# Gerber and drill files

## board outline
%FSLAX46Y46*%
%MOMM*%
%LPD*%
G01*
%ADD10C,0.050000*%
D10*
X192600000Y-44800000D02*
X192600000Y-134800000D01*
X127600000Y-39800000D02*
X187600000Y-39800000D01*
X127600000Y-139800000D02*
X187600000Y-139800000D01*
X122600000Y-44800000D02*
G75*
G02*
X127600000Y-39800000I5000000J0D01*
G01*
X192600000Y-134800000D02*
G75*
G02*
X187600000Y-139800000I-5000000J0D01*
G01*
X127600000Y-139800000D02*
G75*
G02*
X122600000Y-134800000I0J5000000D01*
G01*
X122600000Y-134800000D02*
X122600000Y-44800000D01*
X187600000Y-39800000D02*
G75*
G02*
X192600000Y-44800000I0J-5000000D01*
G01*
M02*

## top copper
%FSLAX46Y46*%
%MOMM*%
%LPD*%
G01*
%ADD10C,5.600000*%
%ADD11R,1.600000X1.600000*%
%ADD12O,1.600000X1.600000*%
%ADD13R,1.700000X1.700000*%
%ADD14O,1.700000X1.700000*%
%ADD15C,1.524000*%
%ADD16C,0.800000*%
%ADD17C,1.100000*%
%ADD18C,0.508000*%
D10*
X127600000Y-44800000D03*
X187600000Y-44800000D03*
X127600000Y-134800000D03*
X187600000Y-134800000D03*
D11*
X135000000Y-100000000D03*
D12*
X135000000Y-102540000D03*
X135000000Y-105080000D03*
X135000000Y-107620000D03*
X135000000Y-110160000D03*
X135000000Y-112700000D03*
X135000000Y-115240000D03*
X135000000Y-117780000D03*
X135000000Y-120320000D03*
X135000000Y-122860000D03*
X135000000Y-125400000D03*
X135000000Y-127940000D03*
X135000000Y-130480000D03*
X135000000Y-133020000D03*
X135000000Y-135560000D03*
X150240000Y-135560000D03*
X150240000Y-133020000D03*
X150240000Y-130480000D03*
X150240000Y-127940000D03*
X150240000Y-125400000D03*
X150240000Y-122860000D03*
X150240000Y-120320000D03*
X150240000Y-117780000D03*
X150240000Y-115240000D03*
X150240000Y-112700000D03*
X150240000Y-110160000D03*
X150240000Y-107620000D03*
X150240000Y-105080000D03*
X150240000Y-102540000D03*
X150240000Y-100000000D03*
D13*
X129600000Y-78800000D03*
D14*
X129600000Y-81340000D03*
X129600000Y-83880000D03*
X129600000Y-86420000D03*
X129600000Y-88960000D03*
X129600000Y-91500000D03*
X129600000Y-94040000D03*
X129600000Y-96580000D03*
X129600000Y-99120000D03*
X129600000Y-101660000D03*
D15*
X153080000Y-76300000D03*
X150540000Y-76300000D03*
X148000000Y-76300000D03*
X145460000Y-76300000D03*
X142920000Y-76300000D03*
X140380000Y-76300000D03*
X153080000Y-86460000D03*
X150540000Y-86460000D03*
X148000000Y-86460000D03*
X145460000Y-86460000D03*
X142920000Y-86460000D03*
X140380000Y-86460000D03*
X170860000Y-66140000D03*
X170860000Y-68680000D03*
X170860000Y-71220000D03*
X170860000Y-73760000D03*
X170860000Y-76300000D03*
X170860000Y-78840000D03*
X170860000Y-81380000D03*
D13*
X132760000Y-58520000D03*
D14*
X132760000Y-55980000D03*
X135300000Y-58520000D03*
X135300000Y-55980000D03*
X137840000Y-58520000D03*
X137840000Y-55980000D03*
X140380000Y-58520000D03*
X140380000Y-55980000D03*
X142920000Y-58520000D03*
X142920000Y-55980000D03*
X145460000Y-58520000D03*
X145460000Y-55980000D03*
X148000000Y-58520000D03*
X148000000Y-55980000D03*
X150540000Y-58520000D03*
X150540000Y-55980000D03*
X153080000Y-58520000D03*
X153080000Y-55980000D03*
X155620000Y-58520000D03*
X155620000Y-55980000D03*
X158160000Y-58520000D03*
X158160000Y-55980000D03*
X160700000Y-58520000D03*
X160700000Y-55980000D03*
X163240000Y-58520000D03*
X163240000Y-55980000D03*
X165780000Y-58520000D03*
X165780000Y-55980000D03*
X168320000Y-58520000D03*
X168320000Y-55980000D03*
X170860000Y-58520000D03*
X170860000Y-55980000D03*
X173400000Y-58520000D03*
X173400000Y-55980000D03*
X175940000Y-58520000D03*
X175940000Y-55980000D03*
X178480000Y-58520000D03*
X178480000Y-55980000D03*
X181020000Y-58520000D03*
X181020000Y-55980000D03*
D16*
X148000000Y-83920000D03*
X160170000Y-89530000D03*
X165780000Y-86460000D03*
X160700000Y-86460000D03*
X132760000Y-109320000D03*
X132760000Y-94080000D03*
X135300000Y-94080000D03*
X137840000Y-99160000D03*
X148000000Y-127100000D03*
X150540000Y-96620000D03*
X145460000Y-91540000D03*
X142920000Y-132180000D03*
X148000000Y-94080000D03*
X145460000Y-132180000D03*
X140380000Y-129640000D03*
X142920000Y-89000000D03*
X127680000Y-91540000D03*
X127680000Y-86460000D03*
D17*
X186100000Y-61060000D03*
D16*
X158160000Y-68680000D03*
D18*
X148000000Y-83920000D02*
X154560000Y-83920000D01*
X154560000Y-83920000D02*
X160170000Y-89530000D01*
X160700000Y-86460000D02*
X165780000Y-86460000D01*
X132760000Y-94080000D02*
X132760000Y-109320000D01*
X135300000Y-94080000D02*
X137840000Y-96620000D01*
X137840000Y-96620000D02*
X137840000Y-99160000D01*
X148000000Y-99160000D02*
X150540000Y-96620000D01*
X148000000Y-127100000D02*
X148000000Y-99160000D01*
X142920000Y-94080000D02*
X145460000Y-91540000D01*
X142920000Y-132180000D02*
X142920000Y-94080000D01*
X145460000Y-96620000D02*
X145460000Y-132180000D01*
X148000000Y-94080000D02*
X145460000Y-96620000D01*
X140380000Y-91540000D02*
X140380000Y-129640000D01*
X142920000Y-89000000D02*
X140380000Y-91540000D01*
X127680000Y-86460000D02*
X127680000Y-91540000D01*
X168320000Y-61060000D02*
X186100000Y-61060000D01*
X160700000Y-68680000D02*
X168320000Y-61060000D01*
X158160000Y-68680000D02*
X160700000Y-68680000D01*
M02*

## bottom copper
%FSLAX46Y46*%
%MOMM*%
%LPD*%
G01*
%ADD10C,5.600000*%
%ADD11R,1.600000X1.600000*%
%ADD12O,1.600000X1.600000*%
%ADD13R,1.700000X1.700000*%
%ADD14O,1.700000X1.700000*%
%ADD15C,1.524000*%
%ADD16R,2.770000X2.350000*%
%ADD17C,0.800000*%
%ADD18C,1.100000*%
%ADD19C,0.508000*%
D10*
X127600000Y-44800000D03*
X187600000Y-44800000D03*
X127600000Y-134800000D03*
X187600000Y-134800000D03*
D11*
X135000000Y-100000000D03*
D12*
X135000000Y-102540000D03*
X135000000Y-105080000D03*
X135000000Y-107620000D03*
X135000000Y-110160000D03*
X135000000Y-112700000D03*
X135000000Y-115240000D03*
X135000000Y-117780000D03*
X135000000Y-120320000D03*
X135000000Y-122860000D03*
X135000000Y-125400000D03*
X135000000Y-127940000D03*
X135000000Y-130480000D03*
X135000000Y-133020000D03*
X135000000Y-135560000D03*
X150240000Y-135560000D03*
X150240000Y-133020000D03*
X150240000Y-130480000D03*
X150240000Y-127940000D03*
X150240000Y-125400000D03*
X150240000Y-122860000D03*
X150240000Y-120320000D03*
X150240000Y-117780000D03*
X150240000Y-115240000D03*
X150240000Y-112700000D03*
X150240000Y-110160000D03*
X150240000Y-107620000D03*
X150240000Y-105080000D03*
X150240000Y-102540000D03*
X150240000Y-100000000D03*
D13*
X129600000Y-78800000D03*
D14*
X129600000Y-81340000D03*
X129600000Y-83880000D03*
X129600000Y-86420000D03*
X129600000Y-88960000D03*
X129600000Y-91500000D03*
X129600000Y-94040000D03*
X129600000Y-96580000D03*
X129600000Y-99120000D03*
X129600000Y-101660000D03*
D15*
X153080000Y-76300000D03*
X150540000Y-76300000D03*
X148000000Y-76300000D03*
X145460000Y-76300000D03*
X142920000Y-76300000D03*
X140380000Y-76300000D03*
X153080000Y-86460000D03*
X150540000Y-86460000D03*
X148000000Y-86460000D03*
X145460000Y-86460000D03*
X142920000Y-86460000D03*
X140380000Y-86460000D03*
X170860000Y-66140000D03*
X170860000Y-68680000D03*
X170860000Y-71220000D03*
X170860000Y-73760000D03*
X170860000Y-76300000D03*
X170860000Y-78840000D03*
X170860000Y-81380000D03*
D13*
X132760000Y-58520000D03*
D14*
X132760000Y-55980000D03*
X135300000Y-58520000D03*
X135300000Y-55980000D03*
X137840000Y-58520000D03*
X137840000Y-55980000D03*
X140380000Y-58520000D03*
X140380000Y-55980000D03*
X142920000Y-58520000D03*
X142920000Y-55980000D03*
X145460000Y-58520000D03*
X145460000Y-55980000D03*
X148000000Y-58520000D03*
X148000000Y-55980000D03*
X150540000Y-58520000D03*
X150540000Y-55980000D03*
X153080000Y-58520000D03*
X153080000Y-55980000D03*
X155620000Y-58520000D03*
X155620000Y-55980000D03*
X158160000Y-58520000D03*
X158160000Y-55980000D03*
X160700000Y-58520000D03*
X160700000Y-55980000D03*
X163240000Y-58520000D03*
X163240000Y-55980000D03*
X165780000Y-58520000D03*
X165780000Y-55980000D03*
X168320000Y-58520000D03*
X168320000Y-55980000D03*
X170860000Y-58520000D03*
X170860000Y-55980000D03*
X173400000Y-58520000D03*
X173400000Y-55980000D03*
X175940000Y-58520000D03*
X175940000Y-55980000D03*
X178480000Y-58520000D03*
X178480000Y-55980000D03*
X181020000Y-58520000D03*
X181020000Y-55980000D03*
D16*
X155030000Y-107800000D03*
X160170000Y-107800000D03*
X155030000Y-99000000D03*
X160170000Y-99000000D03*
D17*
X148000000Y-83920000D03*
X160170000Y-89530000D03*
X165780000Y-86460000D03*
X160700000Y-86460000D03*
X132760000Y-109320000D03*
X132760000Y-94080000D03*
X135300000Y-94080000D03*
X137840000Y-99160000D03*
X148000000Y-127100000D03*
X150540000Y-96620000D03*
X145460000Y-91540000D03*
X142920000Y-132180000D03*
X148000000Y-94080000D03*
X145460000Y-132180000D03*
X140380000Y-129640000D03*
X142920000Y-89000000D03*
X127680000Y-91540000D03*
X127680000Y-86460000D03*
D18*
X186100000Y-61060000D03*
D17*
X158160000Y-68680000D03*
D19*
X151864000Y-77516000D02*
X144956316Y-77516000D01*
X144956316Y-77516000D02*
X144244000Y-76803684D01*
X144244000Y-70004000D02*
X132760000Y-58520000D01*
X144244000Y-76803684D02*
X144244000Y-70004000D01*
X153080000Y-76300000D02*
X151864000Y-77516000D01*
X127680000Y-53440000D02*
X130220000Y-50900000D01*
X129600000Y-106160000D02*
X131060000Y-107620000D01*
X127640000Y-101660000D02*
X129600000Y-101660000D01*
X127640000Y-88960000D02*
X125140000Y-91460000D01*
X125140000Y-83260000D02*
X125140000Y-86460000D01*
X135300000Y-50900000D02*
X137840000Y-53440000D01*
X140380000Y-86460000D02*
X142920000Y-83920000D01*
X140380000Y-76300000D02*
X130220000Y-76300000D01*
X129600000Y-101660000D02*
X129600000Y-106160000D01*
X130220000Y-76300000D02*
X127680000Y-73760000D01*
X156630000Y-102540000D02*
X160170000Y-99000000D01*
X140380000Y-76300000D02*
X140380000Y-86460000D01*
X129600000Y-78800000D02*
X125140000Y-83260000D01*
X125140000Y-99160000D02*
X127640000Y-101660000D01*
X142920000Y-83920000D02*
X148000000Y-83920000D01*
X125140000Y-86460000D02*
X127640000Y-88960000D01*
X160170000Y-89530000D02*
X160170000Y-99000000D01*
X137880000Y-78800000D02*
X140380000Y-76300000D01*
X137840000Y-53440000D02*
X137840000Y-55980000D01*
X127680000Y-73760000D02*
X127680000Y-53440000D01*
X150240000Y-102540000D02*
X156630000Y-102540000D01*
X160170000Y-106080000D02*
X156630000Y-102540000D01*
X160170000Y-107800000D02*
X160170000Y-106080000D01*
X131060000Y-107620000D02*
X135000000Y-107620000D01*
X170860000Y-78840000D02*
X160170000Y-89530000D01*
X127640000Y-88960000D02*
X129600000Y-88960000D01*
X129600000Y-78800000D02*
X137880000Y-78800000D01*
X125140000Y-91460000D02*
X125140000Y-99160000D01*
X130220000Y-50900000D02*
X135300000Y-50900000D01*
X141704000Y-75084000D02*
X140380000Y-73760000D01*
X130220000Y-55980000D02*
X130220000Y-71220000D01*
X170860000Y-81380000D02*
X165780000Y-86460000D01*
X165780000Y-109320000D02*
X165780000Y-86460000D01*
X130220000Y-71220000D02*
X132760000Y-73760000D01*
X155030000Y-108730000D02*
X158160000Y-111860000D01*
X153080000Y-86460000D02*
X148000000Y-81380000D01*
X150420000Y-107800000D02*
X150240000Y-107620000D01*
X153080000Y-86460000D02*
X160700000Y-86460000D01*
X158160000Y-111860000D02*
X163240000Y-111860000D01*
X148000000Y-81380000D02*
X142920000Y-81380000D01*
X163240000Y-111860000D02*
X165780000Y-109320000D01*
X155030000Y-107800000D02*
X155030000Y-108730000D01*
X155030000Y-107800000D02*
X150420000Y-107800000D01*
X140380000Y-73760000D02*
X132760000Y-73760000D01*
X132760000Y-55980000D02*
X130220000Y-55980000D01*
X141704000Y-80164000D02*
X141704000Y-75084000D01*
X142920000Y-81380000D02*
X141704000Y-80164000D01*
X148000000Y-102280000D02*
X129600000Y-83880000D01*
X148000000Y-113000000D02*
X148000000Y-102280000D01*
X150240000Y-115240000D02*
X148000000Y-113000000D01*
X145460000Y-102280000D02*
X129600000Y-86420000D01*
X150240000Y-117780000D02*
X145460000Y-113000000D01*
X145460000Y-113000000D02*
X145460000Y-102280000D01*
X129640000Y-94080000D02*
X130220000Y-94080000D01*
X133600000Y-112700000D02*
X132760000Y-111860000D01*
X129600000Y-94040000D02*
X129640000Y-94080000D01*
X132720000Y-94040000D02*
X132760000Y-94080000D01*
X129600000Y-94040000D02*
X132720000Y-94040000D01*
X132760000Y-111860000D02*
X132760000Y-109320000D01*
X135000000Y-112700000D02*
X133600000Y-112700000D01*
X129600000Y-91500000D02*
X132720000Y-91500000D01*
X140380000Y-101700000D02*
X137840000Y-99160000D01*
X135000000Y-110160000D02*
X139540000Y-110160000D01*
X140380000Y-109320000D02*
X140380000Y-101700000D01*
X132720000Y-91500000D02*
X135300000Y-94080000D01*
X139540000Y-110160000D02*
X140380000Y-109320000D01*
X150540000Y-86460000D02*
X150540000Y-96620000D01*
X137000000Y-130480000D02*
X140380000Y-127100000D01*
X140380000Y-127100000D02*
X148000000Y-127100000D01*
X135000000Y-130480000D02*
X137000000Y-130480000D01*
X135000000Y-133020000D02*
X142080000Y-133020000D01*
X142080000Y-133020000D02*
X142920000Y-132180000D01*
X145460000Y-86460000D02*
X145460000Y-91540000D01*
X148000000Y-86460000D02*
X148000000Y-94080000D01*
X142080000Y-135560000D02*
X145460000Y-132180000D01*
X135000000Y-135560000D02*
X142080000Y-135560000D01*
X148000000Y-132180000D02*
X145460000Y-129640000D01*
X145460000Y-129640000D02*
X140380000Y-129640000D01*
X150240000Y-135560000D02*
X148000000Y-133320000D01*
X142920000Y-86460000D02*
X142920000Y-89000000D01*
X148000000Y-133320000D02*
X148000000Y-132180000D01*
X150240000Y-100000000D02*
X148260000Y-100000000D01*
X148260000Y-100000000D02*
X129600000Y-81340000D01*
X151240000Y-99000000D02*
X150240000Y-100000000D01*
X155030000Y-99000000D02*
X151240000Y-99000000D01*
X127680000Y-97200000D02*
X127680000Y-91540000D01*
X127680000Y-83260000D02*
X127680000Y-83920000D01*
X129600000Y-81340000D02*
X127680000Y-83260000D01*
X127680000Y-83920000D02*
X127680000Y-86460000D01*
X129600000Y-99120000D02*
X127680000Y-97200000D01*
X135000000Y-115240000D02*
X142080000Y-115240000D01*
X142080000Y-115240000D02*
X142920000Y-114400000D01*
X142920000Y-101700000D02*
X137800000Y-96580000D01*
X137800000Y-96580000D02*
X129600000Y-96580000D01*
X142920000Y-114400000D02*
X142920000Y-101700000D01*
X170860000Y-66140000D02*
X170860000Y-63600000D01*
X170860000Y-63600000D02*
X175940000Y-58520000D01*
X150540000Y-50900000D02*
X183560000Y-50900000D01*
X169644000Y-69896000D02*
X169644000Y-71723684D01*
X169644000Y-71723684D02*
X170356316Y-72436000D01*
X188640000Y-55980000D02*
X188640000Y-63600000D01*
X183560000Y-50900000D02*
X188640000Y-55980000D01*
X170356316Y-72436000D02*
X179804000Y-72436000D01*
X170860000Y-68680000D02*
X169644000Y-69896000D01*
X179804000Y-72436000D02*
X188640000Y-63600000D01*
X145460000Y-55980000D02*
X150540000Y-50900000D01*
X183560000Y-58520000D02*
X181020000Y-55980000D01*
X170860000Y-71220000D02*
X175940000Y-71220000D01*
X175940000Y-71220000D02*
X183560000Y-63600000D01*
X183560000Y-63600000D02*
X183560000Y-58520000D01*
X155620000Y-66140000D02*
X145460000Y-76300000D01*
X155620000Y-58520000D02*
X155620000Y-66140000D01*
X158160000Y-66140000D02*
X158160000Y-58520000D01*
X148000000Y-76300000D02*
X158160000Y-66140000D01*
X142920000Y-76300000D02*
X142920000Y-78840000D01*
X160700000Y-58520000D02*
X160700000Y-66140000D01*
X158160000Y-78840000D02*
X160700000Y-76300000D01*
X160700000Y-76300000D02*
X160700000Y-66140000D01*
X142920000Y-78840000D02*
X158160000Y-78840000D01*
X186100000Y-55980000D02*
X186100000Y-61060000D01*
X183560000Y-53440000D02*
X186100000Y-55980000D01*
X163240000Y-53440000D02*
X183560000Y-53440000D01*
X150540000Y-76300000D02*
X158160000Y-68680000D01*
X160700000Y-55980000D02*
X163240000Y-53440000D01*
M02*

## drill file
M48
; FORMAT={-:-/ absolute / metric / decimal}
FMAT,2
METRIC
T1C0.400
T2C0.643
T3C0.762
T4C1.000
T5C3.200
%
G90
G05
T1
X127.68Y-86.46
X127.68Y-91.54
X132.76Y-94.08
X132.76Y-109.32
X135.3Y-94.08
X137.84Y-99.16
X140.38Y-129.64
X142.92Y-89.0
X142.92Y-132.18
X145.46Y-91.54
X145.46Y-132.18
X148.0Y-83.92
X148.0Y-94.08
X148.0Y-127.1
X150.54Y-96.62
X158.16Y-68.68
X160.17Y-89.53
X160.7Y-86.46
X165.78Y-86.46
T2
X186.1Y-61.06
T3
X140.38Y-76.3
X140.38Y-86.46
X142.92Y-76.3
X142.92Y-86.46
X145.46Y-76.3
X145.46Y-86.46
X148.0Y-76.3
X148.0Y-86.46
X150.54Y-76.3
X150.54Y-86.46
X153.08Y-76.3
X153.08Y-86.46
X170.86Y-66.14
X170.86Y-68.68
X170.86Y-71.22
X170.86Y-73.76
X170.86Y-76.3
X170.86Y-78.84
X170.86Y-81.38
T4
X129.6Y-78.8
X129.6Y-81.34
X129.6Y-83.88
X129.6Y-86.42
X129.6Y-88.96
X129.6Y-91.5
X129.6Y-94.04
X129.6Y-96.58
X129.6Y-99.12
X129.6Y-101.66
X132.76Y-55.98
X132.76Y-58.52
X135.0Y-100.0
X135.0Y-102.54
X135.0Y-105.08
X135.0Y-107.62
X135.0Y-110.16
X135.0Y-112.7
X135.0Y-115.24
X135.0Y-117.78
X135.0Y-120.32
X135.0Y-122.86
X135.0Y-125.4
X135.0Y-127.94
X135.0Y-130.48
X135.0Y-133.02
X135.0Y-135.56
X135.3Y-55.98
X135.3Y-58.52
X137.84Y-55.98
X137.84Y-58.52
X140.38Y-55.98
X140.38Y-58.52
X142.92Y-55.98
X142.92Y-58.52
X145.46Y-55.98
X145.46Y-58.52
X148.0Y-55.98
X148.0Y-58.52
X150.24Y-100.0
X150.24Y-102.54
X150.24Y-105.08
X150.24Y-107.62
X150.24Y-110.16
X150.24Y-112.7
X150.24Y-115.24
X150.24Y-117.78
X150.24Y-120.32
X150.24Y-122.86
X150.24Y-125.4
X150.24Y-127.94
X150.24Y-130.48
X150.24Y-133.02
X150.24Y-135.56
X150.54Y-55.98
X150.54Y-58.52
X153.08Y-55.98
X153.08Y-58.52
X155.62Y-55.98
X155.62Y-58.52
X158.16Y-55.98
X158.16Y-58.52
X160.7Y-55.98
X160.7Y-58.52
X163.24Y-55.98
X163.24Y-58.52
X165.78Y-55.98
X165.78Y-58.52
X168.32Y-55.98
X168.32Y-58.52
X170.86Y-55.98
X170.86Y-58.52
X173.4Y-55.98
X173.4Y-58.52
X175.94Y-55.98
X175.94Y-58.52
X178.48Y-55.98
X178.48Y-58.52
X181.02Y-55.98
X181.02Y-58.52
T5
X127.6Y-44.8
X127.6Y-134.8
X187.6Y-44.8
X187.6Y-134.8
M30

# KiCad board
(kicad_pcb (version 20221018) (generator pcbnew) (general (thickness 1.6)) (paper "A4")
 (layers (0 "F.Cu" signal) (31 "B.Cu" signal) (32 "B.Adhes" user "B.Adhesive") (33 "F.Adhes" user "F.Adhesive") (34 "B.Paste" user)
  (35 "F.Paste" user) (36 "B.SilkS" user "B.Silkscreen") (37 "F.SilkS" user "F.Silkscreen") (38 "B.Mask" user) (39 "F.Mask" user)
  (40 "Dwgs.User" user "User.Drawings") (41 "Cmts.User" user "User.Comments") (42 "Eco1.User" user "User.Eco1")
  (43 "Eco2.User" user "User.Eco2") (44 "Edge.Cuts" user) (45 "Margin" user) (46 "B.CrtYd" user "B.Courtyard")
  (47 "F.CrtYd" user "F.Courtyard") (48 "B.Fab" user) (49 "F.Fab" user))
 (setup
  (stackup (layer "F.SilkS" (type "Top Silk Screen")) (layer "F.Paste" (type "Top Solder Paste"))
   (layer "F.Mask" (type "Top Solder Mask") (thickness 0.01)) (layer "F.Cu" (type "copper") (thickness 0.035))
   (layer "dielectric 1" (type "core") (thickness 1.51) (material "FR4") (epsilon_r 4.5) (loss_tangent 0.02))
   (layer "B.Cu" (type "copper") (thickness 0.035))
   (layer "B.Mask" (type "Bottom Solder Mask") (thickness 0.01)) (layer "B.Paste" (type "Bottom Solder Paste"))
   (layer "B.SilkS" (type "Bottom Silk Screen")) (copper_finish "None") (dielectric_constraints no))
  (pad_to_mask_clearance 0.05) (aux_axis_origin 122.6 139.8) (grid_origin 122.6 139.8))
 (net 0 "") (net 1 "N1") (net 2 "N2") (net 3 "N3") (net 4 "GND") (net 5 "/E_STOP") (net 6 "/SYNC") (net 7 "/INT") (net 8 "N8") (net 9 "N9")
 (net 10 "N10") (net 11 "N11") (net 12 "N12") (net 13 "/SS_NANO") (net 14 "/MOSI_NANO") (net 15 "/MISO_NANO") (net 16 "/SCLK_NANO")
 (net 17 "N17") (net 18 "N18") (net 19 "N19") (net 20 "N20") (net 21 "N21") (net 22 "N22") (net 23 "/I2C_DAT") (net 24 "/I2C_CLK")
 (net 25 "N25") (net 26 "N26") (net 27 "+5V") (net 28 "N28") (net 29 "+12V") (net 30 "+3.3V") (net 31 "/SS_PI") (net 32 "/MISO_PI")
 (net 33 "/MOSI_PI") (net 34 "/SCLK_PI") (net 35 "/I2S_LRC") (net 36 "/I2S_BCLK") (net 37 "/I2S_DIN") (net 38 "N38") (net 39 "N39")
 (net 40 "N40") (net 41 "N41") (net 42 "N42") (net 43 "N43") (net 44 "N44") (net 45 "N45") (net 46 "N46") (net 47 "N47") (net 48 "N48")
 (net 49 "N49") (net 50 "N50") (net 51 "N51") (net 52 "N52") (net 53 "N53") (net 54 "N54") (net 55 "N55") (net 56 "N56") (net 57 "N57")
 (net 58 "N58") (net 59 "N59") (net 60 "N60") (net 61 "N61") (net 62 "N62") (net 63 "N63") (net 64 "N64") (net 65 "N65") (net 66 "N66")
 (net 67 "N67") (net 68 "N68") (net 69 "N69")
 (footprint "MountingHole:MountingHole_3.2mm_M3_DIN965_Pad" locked (layer "F.Cu") (at 127.6 44.8)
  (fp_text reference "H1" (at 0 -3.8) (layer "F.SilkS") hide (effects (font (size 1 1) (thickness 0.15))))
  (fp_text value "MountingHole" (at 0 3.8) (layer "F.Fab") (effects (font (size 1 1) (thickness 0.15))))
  (pad "1" thru_hole circle locked (at 0 0) (size 5.6 5.6) (drill 3.2) (layers "*.Cu" "*.Mask")))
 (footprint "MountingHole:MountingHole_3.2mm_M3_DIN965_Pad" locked (layer "F.Cu") (at 187.6 44.8)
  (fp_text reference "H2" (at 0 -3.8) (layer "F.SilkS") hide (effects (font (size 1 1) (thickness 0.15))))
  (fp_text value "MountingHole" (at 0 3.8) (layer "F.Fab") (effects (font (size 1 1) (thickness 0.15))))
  (pad "1" thru_hole circle locked (at 0 0) (size 5.6 5.6) (drill 3.2) (layers "*.Cu" "*.Mask")))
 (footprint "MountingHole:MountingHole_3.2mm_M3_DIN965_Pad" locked (layer "F.Cu") (at 127.6 134.8)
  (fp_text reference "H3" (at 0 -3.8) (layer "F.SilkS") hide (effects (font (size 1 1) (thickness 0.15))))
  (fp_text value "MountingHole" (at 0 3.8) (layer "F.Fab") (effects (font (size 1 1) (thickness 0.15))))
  (pad "1" thru_hole circle locked (at 0 0) (size 5.6 5.6) (drill 3.2) (layers "*.Cu" "*.Mask")))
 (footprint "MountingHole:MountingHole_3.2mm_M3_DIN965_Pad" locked (layer "F.Cu") (at 187.6 134.8)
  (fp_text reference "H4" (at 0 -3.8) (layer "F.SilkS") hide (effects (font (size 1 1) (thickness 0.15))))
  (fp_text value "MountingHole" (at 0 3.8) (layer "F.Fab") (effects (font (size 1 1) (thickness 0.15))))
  (pad "1" thru_hole circle locked (at 0 0) (size 5.6 5.6) (drill 3.2) (layers "*.Cu" "*.Mask")))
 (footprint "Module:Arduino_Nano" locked (layer "F.Cu") (at 135 100)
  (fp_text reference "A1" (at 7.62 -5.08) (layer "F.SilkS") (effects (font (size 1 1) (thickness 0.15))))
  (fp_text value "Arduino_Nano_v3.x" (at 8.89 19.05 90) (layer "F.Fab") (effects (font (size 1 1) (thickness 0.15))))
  (pad "1" thru_hole rect locked (at 0 0) (size 1.6 1.6) (drill 1) (layers "*.Cu" "*.Mask") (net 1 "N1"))
  (pad "2" thru_hole oval locked (at 0 2.54) (size 1.6 1.6) (drill 1) (layers "*.Cu" "*.Mask") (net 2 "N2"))
  (pad "3" thru_hole oval locked (at 0 5.08) (size 1.6 1.6) (drill 1) (layers "*.Cu" "*.Mask") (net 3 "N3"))
  (pad "4" thru_hole oval locked (at 0 7.62) (size 1.6 1.6) (drill 1) (layers "*.Cu" "*.Mask") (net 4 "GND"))
  (pad "5" thru_hole oval locked (at 0 10.16) (size 1.6 1.6) (drill 1) (layers "*.Cu" "*.Mask") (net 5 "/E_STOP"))
  (pad "6" thru_hole oval locked (at 0 12.7) (size 1.6 1.6) (drill 1) (layers "*.Cu" "*.Mask") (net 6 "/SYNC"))
  (pad "7" thru_hole oval locked (at 0 15.24) (size 1.6 1.6) (drill 1) (layers "*.Cu" "*.Mask") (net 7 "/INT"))
  (pad "8" thru_hole oval locked (at 0 17.78) (size 1.6 1.6) (drill 1) (layers "*.Cu" "*.Mask") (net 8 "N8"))
  (pad "9" thru_hole oval locked (at 0 20.32) (size 1.6 1.6) (drill 1) (layers "*.Cu" "*.Mask") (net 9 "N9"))
  (pad "10" thru_hole oval locked (at 0 22.86) (size 1.6 1.6) (drill 1) (layers "*.Cu" "*.Mask") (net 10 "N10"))
  (pad "11" thru_hole oval locked (at 0 25.4) (size 1.6 1.6) (drill 1) (layers "*.Cu" "*.Mask") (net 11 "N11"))
  (pad "12" thru_hole oval locked (at 0 27.94) (size 1.6 1.6) (drill 1) (layers "*.Cu" "*.Mask") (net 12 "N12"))
  (pad "13" thru_hole oval locked (at 0 30.48) (size 1.6 1.6) (drill 1) (layers "*.Cu" "*.Mask") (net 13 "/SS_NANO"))
  (pad "14" thru_hole oval locked (at 0 33.02) (size 1.6 1.6) (drill 1) (layers "*.Cu" "*.Mask") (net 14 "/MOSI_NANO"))
  (pad "15" thru_hole oval locked (at 0 35.56) (size 1.6 1.6) (drill 1) (layers "*.Cu" "*.Mask") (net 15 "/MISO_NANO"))
  (pad "16" thru_hole oval locked (at 15.24 35.56) (size 1.6 1.6) (drill 1) (layers "*.Cu" "*.Mask") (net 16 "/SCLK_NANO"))
  (pad "17" thru_hole oval locked (at 15.24 33.02) (size 1.6 1.6) (drill 1) (layers "*.Cu" "*.Mask") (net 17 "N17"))
  (pad "18" thru_hole oval locked (at 15.24 30.48) (size 1.6 1.6) (drill 1) (layers "*.Cu" "*.Mask") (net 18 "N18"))
  (pad "19" thru_hole oval locked (at 15.24 27.94) (size 1.6 1.6) (drill 1) (layers "*.Cu" "*.Mask") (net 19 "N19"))
  (pad "20" thru_hole oval locked (at 15.24 25.4) (size 1.6 1.6) (drill 1) (layers "*.Cu" "*.Mask") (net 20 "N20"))
  (pad "21" thru_hole oval locked (at 15.24 22.86) (size 1.6 1.6) (drill 1) (layers "*.Cu" "*.Mask") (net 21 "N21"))
  (pad "22" thru_hole oval locked (at 15.24 20.32) (size 1.6 1.6) (drill 1) (layers "*.Cu" "*.Mask") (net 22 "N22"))
  (pad "23" thru_hole oval locked (at 15.24 17.78) (size 1.6 1.6) (drill 1) (layers "*.Cu" "*.Mask") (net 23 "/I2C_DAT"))
  (pad "24" thru_hole oval locked (at 15.24 15.24) (size 1.6 1.6) (drill 1) (layers "*.Cu" "*.Mask") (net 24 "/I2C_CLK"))
  (pad "25" thru_hole oval locked (at 15.24 12.7) (size 1.6 1.6) (drill 1) (layers "*.Cu" "*.Mask") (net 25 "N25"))
  (pad "26" thru_hole oval locked (at 15.24 10.16) (size 1.6 1.6) (drill 1) (layers "*.Cu" "*.Mask") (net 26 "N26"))
  (pad "27" thru_hole oval locked (at 15.24 7.62) (size 1.6 1.6) (drill 1) (layers "*.Cu" "*.Mask") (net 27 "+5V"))
  (pad "28" thru_hole oval locked (at 15.24 5.08) (size 1.6 1.6) (drill 1) (layers "*.Cu" "*.Mask") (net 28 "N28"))
  (pad "29" thru_hole oval locked (at 15.24 2.54) (size 1.6 1.6) (drill 1) (layers "*.Cu" "*.Mask") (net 4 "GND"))
  (pad "30" thru_hole oval locked (at 15.24 0) (size 1.6 1.6) (drill 1) (layers "*.Cu" "*.Mask") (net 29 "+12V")))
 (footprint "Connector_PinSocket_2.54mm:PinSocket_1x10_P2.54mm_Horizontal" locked (layer "F.Cu") (at 129.6 78.8)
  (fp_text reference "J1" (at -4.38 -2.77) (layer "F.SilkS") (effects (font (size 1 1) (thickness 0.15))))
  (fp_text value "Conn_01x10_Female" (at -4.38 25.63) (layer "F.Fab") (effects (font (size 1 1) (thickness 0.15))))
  (pad "1" thru_hole rect locked (at 0 0) (size 1.7 1.7) (drill 1) (layers "*.Cu" "*.Mask") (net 4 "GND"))
  (pad "2" thru_hole oval locked (at 0 2.54) (size 1.7 1.7) (drill 1) (layers "*.Cu" "*.Mask") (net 29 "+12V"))
  (pad "3" thru_hole oval locked (at 0 5.08) (size 1.7 1.7) (drill 1) (layers "*.Cu" "*.Mask") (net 24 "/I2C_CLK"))
  (pad "4" thru_hole oval locked (at 0 7.62) (size 1.7 1.7) (drill 1) (layers "*.Cu" "*.Mask") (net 23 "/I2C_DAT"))
  (pad "5" thru_hole oval locked (at 0 10.16) (size 1.7 1.7) (drill 1) (layers "*.Cu" "*.Mask") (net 4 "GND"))
  (pad "6" thru_hole oval locked (at 0 12.7) (size 1.7 1.7) (drill 1) (layers "*.Cu" "*.Mask") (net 5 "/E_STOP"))
  (pad "7" thru_hole oval locked (at 0 15.24) (size 1.7 1.7) (drill 1) (layers "*.Cu" "*.Mask") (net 6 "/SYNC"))
  (pad "8" thru_hole oval locked (at 0 17.78) (size 1.7 1.7) (drill 1) (layers "*.Cu" "*.Mask") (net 7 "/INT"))
  (pad "9" thru_hole oval locked (at 0 20.32) (size 1.7 1.7) (drill 1) (layers "*.Cu" "*.Mask") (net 29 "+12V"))
  (pad "10" thru_hole oval locked (at 0 22.86) (size 1.7 1.7) (drill 1) (layers "*.Cu" "*.Mask") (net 4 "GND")))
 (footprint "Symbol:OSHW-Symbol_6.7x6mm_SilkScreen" (layer "F.Cu") (at 166.6 135.8)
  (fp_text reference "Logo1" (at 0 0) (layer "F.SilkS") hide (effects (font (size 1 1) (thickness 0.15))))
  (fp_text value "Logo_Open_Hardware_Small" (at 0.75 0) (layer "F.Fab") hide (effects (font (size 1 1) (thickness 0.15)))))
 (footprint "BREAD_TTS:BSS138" (layer "F.Cu") (at 145.46 73.76 180)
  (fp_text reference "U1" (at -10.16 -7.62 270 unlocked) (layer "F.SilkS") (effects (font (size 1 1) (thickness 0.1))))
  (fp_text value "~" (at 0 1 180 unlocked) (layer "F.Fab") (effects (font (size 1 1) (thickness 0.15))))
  (pad "1" thru_hole circle (at -7.62 -2.54 180) (size 1.524 1.524) (drill 0.762) (layers "*.Cu" "*.Mask") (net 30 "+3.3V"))
  (pad "2" thru_hole circle (at -5.08 -2.54 180) (size 1.524 1.524) (drill 0.762) (layers "*.Cu" "*.Mask") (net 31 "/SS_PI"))
  (pad "3" thru_hole circle (at -2.54 -2.54 180) (size 1.524 1.524) (drill 0.762) (layers "*.Cu" "*.Mask") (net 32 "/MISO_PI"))
  (pad "4" thru_hole circle (at 0 -2.54 180) (size 1.524 1.524) (drill 0.762) (layers "*.Cu" "*.Mask") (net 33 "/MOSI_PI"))
  (pad "5" thru_hole circle (at 2.54 -2.54 180) (size 1.524 1.524) (drill 0.762) (layers "*.Cu" "*.Mask") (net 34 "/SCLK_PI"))
  (pad "6" thru_hole circle (at 5.08 -2.54 180) (size 1.524 1.524) (drill 0.762) (layers "*.Cu" "*.Mask") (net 4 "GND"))
  (pad "7" thru_hole circle (at -7.62 -12.7 180) (size 1.524 1.524) (drill 0.762) (layers "*.Cu" "*.Mask") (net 27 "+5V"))
  (pad "8" thru_hole circle (at -5.08 -12.7 180) (size 1.524 1.524) (drill 0.762) (layers "*.Cu" "*.Mask") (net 13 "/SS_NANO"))
  (pad "9" thru_hole circle (at -2.54 -12.7 180) (size 1.524 1.524) (drill 0.762) (layers "*.Cu" "*.Mask") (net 15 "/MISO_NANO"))
  (pad "10" thru_hole circle (at 0 -12.7 180) (size 1.524 1.524) (drill 0.762) (layers "*.Cu" "*.Mask") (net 14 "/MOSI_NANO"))
  (pad "11" thru_hole circle (at 2.54 -12.7 180) (size 1.524 1.524) (drill 0.762) (layers "*.Cu" "*.Mask") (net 16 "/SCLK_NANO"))
  (pad "12" thru_hole circle (at 5.08 -12.7 180) (size 1.524 1.524) (drill 0.762) (layers "*.Cu" "*.Mask") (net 4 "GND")))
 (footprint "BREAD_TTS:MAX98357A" (layer "F.Cu") (at 168.32 73.76 -90)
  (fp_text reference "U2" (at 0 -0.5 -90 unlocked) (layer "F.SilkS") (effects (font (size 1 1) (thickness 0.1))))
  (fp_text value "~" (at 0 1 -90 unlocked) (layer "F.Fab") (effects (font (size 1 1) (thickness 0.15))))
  (pad "1" thru_hole circle (at -7.62 -2.54 270) (size 1.524 1.524) (drill 0.762) (layers "*.Cu" "*.Mask") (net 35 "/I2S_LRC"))
  (pad "2" thru_hole circle (at -5.08 -2.54 270) (size 1.524 1.524) (drill 0.762) (layers "*.Cu" "*.Mask") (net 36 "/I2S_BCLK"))
  (pad "3" thru_hole circle (at -2.54 -2.54 270) (size 1.524 1.524) (drill 0.762) (layers "*.Cu" "*.Mask") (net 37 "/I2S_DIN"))
  (pad "4" thru_hole circle (at 0 -2.54 270) (size 1.524 1.524) (drill 0.762) (layers "*.Cu" "*.Mask") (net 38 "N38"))
  (pad "5" thru_hole circle (at 2.54 -2.54 270) (size 1.524 1.524) (drill 0.762) (layers "*.Cu" "*.Mask") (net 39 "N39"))
  (pad "6" thru_hole circle (at 5.08 -2.54 270) (size 1.524 1.524) (drill 0.762) (layers "*.Cu" "*.Mask") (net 4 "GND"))
  (pad "7" thru_hole circle (at 7.62 -2.54 270) (size 1.524 1.524) (drill 0.762) (layers "*.Cu" "*.Mask") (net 27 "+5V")))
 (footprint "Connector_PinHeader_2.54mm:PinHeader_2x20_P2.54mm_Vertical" (layer "F.Cu") (at 132.76 58.52 90)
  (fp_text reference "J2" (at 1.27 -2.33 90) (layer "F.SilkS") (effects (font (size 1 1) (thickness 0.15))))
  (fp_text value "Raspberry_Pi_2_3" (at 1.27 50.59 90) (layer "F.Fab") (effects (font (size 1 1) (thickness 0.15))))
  (pad "1" thru_hole rect (at 0 0 90) (size 1.7 1.7) (drill 1) (layers "*.Cu" "*.Mask") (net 30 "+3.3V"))
  (pad "2" thru_hole oval (at 2.54 0 90) (size 1.7 1.7) (drill 1) (layers "*.Cu" "*.Mask") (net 27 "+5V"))
  (pad "3" thru_hole oval (at 0 2.54 90) (size 1.7 1.7) (drill 1) (layers "*.Cu" "*.Mask") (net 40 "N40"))
  (pad "4" thru_hole oval (at 2.54 2.54 90) (size 1.7 1.7) (drill 1) (layers "*.Cu" "*.Mask") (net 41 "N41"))
  (pad "5" thru_hole oval (at 0 5.08 90) (size 1.7 1.7) (drill 1) (layers "*.Cu" "*.Mask") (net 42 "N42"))
  (pad "6" thru_hole oval (at 2.54 5.08 90) (size 1.7 1.7) (drill 1) (layers "*.Cu" "*.Mask") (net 4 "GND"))
  (pad "7" thru_hole oval (at 0 7.62 90) (size 1.7 1.7) (drill 1) (layers "*.Cu" "*.Mask") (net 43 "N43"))
  (pad "8" thru_hole oval (at 2.54 7.62 90) (size 1.7 1.7) (drill 1) (layers "*.Cu" "*.Mask") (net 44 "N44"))
  (pad "9" thru_hole oval (at 0 10.16 90) (size 1.7 1.7) (drill 1) (layers "*.Cu" "*.Mask") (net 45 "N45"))
  (pad "10" thru_hole oval (at 2.54 10.16 90) (size 1.7 1.7) (drill 1) (layers "*.Cu" "*.Mask") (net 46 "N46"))
  (pad "11" thru_hole oval (at 0 12.7 90) (size 1.7 1.7) (drill 1) (layers "*.Cu" "*.Mask") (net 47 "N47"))
  (pad "12" thru_hole oval (at 2.54 12.7 90) (size 1.7 1.7) (drill 1) (layers "*.Cu" "*.Mask") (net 36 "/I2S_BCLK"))
  (pad "13" thru_hole oval (at 0 15.24 90) (size 1.7 1.7) (drill 1) (layers "*.Cu" "*.Mask") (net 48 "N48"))
  (pad "14" thru_hole oval (at 2.54 15.24 90) (size 1.7 1.7) (drill 1) (layers "*.Cu" "*.Mask") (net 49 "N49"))
  (pad "15" thru_hole oval (at 0 17.78 90) (size 1.7 1.7) (drill 1) (layers "*.Cu" "*.Mask") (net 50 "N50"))
  (pad "16" thru_hole oval (at 2.54 17.78 90) (size 1.7 1.7) (drill 1) (layers "*.Cu" "*.Mask") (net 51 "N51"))
  (pad "17" thru_hole oval (at 0 20.32 90) (size 1.7 1.7) (drill 1) (layers "*.Cu" "*.Mask") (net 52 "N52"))
  (pad "18" thru_hole oval (at 2.54 20.32 90) (size 1.7 1.7) (drill 1) (layers "*.Cu" "*.Mask") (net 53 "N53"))
  (pad "19" thru_hole oval (at 0 22.86 90) (size 1.7 1.7) (drill 1) (layers "*.Cu" "*.Mask") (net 33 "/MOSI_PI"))
  (pad "20" thru_hole oval (at 2.54 22.86 90) (size 1.7 1.7) (drill 1) (layers "*.Cu" "*.Mask") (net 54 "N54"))
  (pad "21" thru_hole oval (at 0 25.4 90) (size 1.7 1.7) (drill 1) (layers "*.Cu" "*.Mask") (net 32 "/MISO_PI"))
  (pad "22" thru_hole oval (at 2.54 25.4 90) (size 1.7 1.7) (drill 1) (layers "*.Cu" "*.Mask") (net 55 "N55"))
  (pad "23" thru_hole oval (at 0 27.94 90) (size 1.7 1.7) (drill 1) (layers "*.Cu" "*.Mask") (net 34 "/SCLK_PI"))
  (pad "24" thru_hole oval (at 2.54 27.94 90) (size 1.7 1.7) (drill 1) (layers "*.Cu" "*.Mask") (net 31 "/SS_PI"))
  (pad "25" thru_hole oval (at 0 30.48 90) (size 1.7 1.7) (drill 1) (layers "*.Cu" "*.Mask") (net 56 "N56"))
  (pad "26" thru_hole oval (at 2.54 30.48 90) (size 1.7 1.7) (drill 1) (layers "*.Cu" "*.Mask") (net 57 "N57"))
  (pad "27" thru_hole oval (at 0 33.02 90) (size 1.7 1.7) (drill 1) (layers "*.Cu" "*.Mask") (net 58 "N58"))
  (pad "28" thru_hole oval (at 2.54 33.02 90) (size 1.7 1.7) (drill 1) (layers "*.Cu" "*.Mask") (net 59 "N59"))
  (pad "29" thru_hole oval (at 0 35.56 90) (size 1.7 1.7) (drill 1) (layers "*.Cu" "*.Mask") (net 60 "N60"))
  (pad "30" thru_hole oval (at 2.54 35.56 90) (size 1.7 1.7) (drill 1) (layers "*.Cu" "*.Mask") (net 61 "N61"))
  (pad "31" thru_hole oval (at 0 38.1 90) (size 1.7 1.7) (drill 1) (layers "*.Cu" "*.Mask") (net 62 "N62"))
  (pad "32" thru_hole oval (at 2.54 38.1 90) (size 1.7 1.7) (drill 1) (layers "*.Cu" "*.Mask") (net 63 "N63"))
  (pad "33" thru_hole oval (at 0 40.64 90) (size 1.7 1.7) (drill 1) (layers "*.Cu" "*.Mask") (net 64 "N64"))
  (pad "34" thru_hole oval (at 2.54 40.64 90) (size 1.7 1.7) (drill 1) (layers "*.Cu" "*.Mask") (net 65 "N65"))
  (pad "35" thru_hole oval (at 0 43.18 90) (size 1.7 1.7) (drill 1) (layers "*.Cu" "*.Mask") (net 35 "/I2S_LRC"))
  (pad "36" thru_hole oval (at 2.54 43.18 90) (size 1.7 1.7) (drill 1) (layers "*.Cu" "*.Mask") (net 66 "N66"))
  (pad "37" thru_hole oval (at 0 45.72 90) (size 1.7 1.7) (drill 1) (layers "*.Cu" "*.Mask") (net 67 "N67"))
  (pad "38" thru_hole oval (at 2.54 45.72 90) (size 1.7 1.7) (drill 1) (layers "*.Cu" "*.Mask") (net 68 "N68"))
  (pad "39" thru_hole oval (at 0 48.26 90) (size 1.7 1.7) (drill 1) (layers "*.Cu" "*.Mask") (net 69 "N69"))
  (pad "40" thru_hole oval (at 2.54 48.26 90) (size 1.7 1.7) (drill 1) (layers "*.Cu" "*.Mask") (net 37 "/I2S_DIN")))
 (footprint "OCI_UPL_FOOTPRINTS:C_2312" (layer "B.Cu") (at 157.6 107.8)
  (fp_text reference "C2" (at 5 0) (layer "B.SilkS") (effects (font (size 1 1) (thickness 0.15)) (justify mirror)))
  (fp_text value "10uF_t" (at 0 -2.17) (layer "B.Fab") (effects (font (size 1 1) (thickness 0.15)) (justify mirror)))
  (pad "1" smd rect (at -2.57 0) (size 2.77 2.35) (layers "B.Cu" "B.Paste" "B.Mask") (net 27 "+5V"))
  (pad "2" smd rect (at 2.57 0) (size 2.77 2.35) (layers "B.Cu" "B.Paste" "B.Mask") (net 4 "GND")))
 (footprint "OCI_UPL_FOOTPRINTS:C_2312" (layer "B.Cu") (at 157.6 99)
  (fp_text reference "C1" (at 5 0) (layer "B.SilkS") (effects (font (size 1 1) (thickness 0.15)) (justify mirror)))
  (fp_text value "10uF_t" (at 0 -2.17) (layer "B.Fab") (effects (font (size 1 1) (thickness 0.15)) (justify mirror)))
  (pad "1" smd rect (at -2.57 0) (size 2.77 2.35) (layers "B.Cu" "B.Paste" "B.Mask") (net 29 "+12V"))
  (pad "2" smd rect (at 2.57 0) (size 2.77 2.35) (layers "B.Cu" "B.Paste" "B.Mask") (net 4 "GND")))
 (gr_line (start 192.6 44.8) (end 192.6 134.8) (stroke (width 0.05) (type solid)) (layer "Edge.Cuts"))
 (gr_line (start 127.6 39.8) (end 187.6 39.8) (stroke (width 0.05) (type solid)) (layer "Edge.Cuts"))
 (gr_line (start 127.6 139.8) (end 187.6 139.8) (stroke (width 0.05) (type solid)) (layer "Edge.Cuts"))
 (gr_arc (start 122.6 44.8) (mid 124.064466 41.264466) (end 127.6 39.8) (stroke (width 0.05) (type solid)) (layer "Edge.Cuts"))
 (gr_arc (start 192.6 134.8) (mid 191.135534 138.335534) (end 187.6 139.8) (stroke (width 0.05) (type solid)) (layer "Edge.Cuts"))
 (gr_arc (start 127.6 139.8) (mid 124.064466 138.335534) (end 122.6 134.8) (stroke (width 0.05) (type solid)) (layer "Edge.Cuts"))
 (gr_line (start 122.6 134.8) (end 122.6 44.8) (stroke (width 0.05) (type solid)) (layer "Edge.Cuts"))
 (gr_arc (start 187.6 39.8) (mid 191.135534 41.264466) (end 192.6 44.8) (stroke (width 0.05) (type solid)) (layer "Edge.Cuts"))
 (segment (start 151.864 77.516) (end 144.956316 77.516) (width 0.508) (layer "B.Cu") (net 30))
 (segment (start 144.956316 77.516) (end 144.244 76.803684) (width 0.508) (layer "B.Cu") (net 30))
 (segment (start 144.244 70.004) (end 132.76 58.52) (width 0.508) (layer "B.Cu") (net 30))
 (segment (start 144.244 76.803684) (end 144.244 70.004) (width 0.508) (layer "B.Cu") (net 30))
 (segment (start 153.08 76.3) (end 151.864 77.516) (width 0.508) (layer "B.Cu") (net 30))
 (segment (start 148 83.92) (end 154.56 83.92) (width 0.508) (layer "F.Cu") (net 4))
 (segment (start 154.56 83.92) (end 160.17 89.53) (width 0.508) (layer "F.Cu") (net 4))
 (via (at 148 83.92) (size 0.8) (drill 0.4) (layers "F.Cu" "B.Cu") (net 4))
 (via (at 160.17 89.53) (size 0.8) (drill 0.4) (layers "F.Cu" "B.Cu") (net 4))
 (segment (start 127.68 53.44) (end 130.22 50.9) (width 0.508) (layer "B.Cu") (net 4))
 (segment (start 129.6 106.16) (end 131.06 107.62) (width 0.508) (layer "B.Cu") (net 4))
 (segment (start 127.64 101.66) (end 129.6 101.66) (width 0.508) (layer "B.Cu") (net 4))
 (segment (start 127.64 88.96) (end 125.14 91.46) (width 0.508) (layer "B.Cu") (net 4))
 (segment (start 125.14 83.26) (end 125.14 86.46) (width 0.508) (layer "B.Cu") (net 4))
 (segment (start 135.3 50.9) (end 137.84 53.44) (width 0.508) (layer "B.Cu") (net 4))
 (segment (start 140.38 86.46) (end 142.92 83.92) (width 0.508) (layer "B.Cu") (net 4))
 (segment (start 140.38 76.3) (end 130.22 76.3) (width 0.508) (layer "B.Cu") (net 4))
 (segment (start 129.6 101.66) (end 129.6 106.16) (width 0.508) (layer "B.Cu") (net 4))
 (segment (start 130.22 76.3) (end 127.68 73.76) (width 0.508) (layer "B.Cu") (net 4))
 (segment (start 156.63 102.54) (end 160.17 99) (width 0.508) (layer "B.Cu") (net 4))
 (segment (start 140.38 76.3) (end 140.38 86.46) (width 0.508) (layer "B.Cu") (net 4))
 (segment (start 129.6 78.8) (end 125.14 83.26) (width 0.508) (layer "B.Cu") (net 4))
 (segment (start 125.14 99.16) (end 127.64 101.66) (width 0.508) (layer "B.Cu") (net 4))
 (segment (start 142.92 83.92) (end 148 83.92) (width 0.508) (layer "B.Cu") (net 4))
 (segment (start 125.14 86.46) (end 127.64 88.96) (width 0.508) (layer "B.Cu") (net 4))
 (segment (start 160.17 89.53) (end 160.17 99) (width 0.508) (layer "B.Cu") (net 4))
 (segment (start 137.88 78.8) (end 140.38 76.3) (width 0.508) (layer "B.Cu") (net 4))
 (segment (start 137.84 53.44) (end 137.84 55.98) (width 0.508) (layer "B.Cu") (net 4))
 (segment (start 127.68 73.76) (end 127.68 53.44) (width 0.508) (layer "B.Cu") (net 4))
 (segment (start 150.24 102.54) (end 156.63 102.54) (width 0.508) (layer "B.Cu") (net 4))
 (segment (start 160.17 106.08) (end 156.63 102.54) (width 0.508) (layer "B.Cu") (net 4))
 (segment (start 160.17 107.8) (end 160.17 106.08) (width 0.508) (layer "B.Cu") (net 4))
 (segment (start 131.06 107.62) (end 135 107.62) (width 0.508) (layer "B.Cu") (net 4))
 (segment (start 170.86 78.84) (end 160.17 89.53) (width 0.508) (layer "B.Cu") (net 4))
 (segment (start 127.64 88.96) (end 129.6 88.96) (width 0.508) (layer "B.Cu") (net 4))
 (segment (start 129.6 78.8) (end 137.88 78.8) (width 0.508) (layer "B.Cu") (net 4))
 (segment (start 125.14 91.46) (end 125.14 99.16) (width 0.508) (layer "B.Cu") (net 4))
 (segment (start 130.22 50.9) (end 135.3 50.9) (width 0.508) (layer "B.Cu") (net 4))
 (segment (start 160.7 86.46) (end 165.78 86.46) (width 0.508) (layer "F.Cu") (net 27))
 (via (at 165.78 86.46) (size 0.8) (drill 0.4) (layers "F.Cu" "B.Cu") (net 27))
 (via (at 160.7 86.46) (size 0.8) (drill 0.4) (layers "F.Cu" "B.Cu") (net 27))
 (segment (start 141.704 75.084) (end 140.38 73.76) (width 0.508) (layer "B.Cu") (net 27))
 (segment (start 130.22 55.98) (end 130.22 71.22) (width 0.508) (layer "B.Cu") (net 27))
 (segment (start 170.86 81.38) (end 165.78 86.46) (width 0.508) (layer "B.Cu") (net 27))
 (segment (start 165.78 109.32) (end 165.78 86.46) (width 0.508) (layer "B.Cu") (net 27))
 (segment (start 130.22 71.22) (end 132.76 73.76) (width 0.508) (layer "B.Cu") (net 27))
 (segment (start 155.03 108.73) (end 158.16 111.86) (width 0.508) (layer "B.Cu") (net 27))
 (segment (start 153.08 86.46) (end 148 81.38) (width 0.508) (layer "B.Cu") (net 27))
 (segment (start 150.42 107.8) (end 150.24 107.62) (width 0.508) (layer "B.Cu") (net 27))
 (segment (start 153.08 86.46) (end 160.7 86.46) (width 0.508) (layer "B.Cu") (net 27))
 (segment (start 158.16 111.86) (end 163.24 111.86) (width 0.508) (layer "B.Cu") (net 27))
 (segment (start 148 81.38) (end 142.92 81.38) (width 0.508) (layer "B.Cu") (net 27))
 (segment (start 163.24 111.86) (end 165.78 109.32) (width 0.508) (layer "B.Cu") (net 27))
 (segment (start 155.03 107.8) (end 155.03 108.73) (width 0.508) (layer "B.Cu") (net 27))
 (segment (start 155.03 107.8) (end 150.42 107.8) (width 0.508) (layer "B.Cu") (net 27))
 (segment (start 140.38 73.76) (end 132.76 73.76) (width 0.508) (layer "B.Cu") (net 27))
 (segment (start 132.76 55.98) (end 130.22 55.98) (width 0.508) (layer "B.Cu") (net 27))
 (segment (start 141.704 80.164) (end 141.704 75.084) (width 0.508) (layer "B.Cu") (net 27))
 (segment (start 142.92 81.38) (end 141.704 80.164) (width 0.508) (layer "B.Cu") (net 27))
 (segment (start 148 102.28) (end 129.6 83.88) (width 0.508) (layer "B.Cu") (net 24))
 (segment (start 148 113) (end 148 102.28) (width 0.508) (layer "B.Cu") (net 24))
 (segment (start 150.24 115.24) (end 148 113) (width 0.508) (layer "B.Cu") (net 24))
 (segment (start 145.46 102.28) (end 129.6 86.42) (width 0.508) (layer "B.Cu") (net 23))
 (segment (start 150.24 117.78) (end 145.46 113) (width 0.508) (layer "B.Cu") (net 23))
 (segment (start 145.46 113) (end 145.46 102.28) (width 0.508) (layer "B.Cu") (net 23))
 (segment (start 132.76 94.08) (end 132.76 109.32) (width 0.508) (layer "F.Cu") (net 6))
 (via (at 132.76 109.32) (size 0.8) (drill 0.4) (layers "F.Cu" "B.Cu") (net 6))
 (via (at 132.76 94.08) (size 0.8) (drill 0.4) (layers "F.Cu" "B.Cu") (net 6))
 (segment (start 129.64 94.08) (end 130.22 94.08) (width 0.508) (layer "B.Cu") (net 6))
 (segment (start 133.6 112.7) (end 132.76 111.86) (width 0.508) (layer "B.Cu") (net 6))
 (segment (start 129.6 94.04) (end 129.64 94.08) (width 0.508) (layer "B.Cu") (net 6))
 (segment (start 132.72 94.04) (end 132.76 94.08) (width 0.508) (layer "B.Cu") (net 6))
 (segment (start 129.6 94.04) (end 132.72 94.04) (width 0.508) (layer "B.Cu") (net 6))
 (segment (start 132.76 111.86) (end 132.76 109.32) (width 0.508) (layer "B.Cu") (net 6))
 (segment (start 135 112.7) (end 133.6 112.7) (width 0.508) (layer "B.Cu") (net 6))
 (segment (start 135.3 94.08) (end 137.84 96.62) (width 0.508) (layer "F.Cu") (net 5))
 (segment (start 137.84 96.62) (end 137.84 99.16) (width 0.508) (layer "F.Cu") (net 5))
 (via (at 135.3 94.08) (size 0.8) (drill 0.4) (layers "F.Cu" "B.Cu") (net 5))
 (via (at 137.84 99.16) (size 0.8) (drill 0.4) (layers "F.Cu" "B.Cu") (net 5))
 (segment (start 129.6 91.5) (end 132.72 91.5) (width 0.508) (layer "B.Cu") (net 5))
 (segment (start 140.38 101.7) (end 137.84 99.16) (width 0.508) (layer "B.Cu") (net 5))
 (segment (start 135 110.16) (end 139.54 110.16) (width 0.508) (layer "B.Cu") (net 5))
 (segment (start 140.38 109.32) (end 140.38 101.7) (width 0.508) (layer "B.Cu") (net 5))
 (segment (start 132.72 91.5) (end 135.3 94.08) (width 0.508) (layer "B.Cu") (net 5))
 (segment (start 139.54 110.16) (end 140.38 109.32) (width 0.508) (layer "B.Cu") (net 5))
 (segment (start 148 99.16) (end 150.54 96.62) (width 0.508) (layer "F.Cu") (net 13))
 (segment (start 148 127.1) (end 148 99.16) (width 0.508) (layer "F.Cu") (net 13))
 (via (at 148 127.1) (size 0.8) (drill 0.4) (layers "F.Cu" "B.Cu") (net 13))
 (via (at 150.54 96.62) (size 0.8) (drill 0.4) (layers "F.Cu" "B.Cu") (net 13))
 (segment (start 150.54 86.46) (end 150.54 96.62) (width 0.508) (layer "B.Cu") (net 13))
 (segment (start 137 130.48) (end 140.38 127.1) (width 0.508) (layer "B.Cu") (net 13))
 (segment (start 140.38 127.1) (end 148 127.1) (width 0.508) (layer "B.Cu") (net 13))
 (segment (start 135 130.48) (end 137 130.48) (width 0.508) (layer "B.Cu") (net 13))
 (segment (start 142.92 94.08) (end 145.46 91.54) (width 0.508) (layer "F.Cu") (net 14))
 (segment (start 142.92 132.18) (end 142.92 94.08) (width 0.508) (layer "F.Cu") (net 14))
 (via (at 145.46 91.54) (size 0.8) (drill 0.4) (layers "F.Cu" "B.Cu") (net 14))
 (via (at 142.92 132.18) (size 0.8) (drill 0.4) (layers "F.Cu" "B.Cu") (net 14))
 (segment (start 135 133.02) (end 142.08 133.02) (width 0.508) (layer "B.Cu") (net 14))
 (segment (start 142.08 133.02) (end 142.92 132.18) (width 0.508) (layer "B.Cu") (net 14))
 (segment (start 145.46 86.46) (end 145.46 91.54) (width 0.508) (layer "B.Cu") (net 14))
 (segment (start 145.46 96.62) (end 145.46 132.18) (width 0.508) (layer "F.Cu") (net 15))
 (segment (start 148 94.08) (end 145.46 96.62) (width 0.508) (layer "F.Cu") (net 15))
 (via (at 148 94.08) (size 0.8) (drill 0.4) (layers "F.Cu" "B.Cu") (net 15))
 (via (at 145.46 132.18) (size 0.8) (drill 0.4) (layers "F.Cu" "B.Cu") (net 15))
 (segment (start 148 86.46) (end 148 94.08) (width 0.508) (layer "B.Cu") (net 15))
 (segment (start 142.08 135.56) (end 145.46 132.18) (width 0.508) (layer "B.Cu") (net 15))
 (segment (start 135 135.56) (end 142.08 135.56) (width 0.508) (layer "B.Cu") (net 15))
 (segment (start 140.38 91.54) (end 140.38 129.64) (width 0.508) (layer "F.Cu") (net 16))
 (segment (start 142.92 89) (end 140.38 91.54) (width 0.508) (layer "F.Cu") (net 16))
 (via (at 140.38 129.64) (size 0.8) (drill 0.4) (layers "F.Cu" "B.Cu") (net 16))
 (via (at 142.92 89) (size 0.8) (drill 0.4) (layers "F.Cu" "B.Cu") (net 16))
 (segment (start 148 132.18) (end 145.46 129.64) (width 0.508) (layer "B.Cu") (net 16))
 (segment (start 145.46 129.64) (end 140.38 129.64) (width 0.508) (layer "B.Cu") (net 16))
 (segment (start 150.24 135.56) (end 148 133.32) (width 0.508) (layer "B.Cu") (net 16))
 (segment (start 142.92 86.46) (end 142.92 89) (width 0.508) (layer "B.Cu") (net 16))
 (segment (start 148 133.32) (end 148 132.18) (width 0.508) (layer "B.Cu") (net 16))
 (segment (start 127.68 86.46) (end 127.68 91.54) (width 0.508) (layer "F.Cu") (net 29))
 (via (at 127.68 91.54) (size 0.8) (drill 0.4) (layers "F.Cu" "B.Cu") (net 29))
 (via (at 127.68 86.46) (size 0.8) (drill 0.4) (layers "F.Cu" "B.Cu") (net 29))
 (segment (start 150.24 100) (end 148.26 100) (width 0.508) (layer "B.Cu") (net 29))
 (segment (start 148.26 100) (end 129.6 81.34) (width 0.508) (layer "B.Cu") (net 29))
 (segment (start 151.24 99) (end 150.24 100) (width 0.508) (layer "B.Cu") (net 29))
 (segment (start 155.03 99) (end 151.24 99) (width 0.508) (layer "B.Cu") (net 29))
 (segment (start 127.68 97.2) (end 127.68 91.54) (width 0.508) (layer "B.Cu") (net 29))
 (segment (start 127.68 83.26) (end 127.68 83.92) (width 0.508) (layer "B.Cu") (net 29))
 (segment (start 129.6 81.34) (end 127.68 83.26) (width 0.508) (layer "B.Cu") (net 29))
 (segment (start 127.68 83.92) (end 127.68 86.46) (width 0.508) (layer "B.Cu") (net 29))
 (segment (start 129.6 99.12) (end 127.68 97.2) (width 0.508) (layer "B.Cu") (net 29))
 (segment (start 135 115.24) (end 142.08 115.24) (width 0.508) (layer "B.Cu") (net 7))
 (segment (start 142.08 115.24) (end 142.92 114.4) (width 0.508) (layer "B.Cu") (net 7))
 (segment (start 142.92 101.7) (end 137.8 96.58) (width 0.508) (layer "B.Cu") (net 7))
 (segment (start 137.8 96.58) (end 129.6 96.58) (width 0.508) (layer "B.Cu") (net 7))
 (segment (start 142.92 114.4) (end 142.92 101.7) (width 0.508) (layer "B.Cu") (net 7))
 (segment (start 170.86 66.14) (end 170.86 63.6) (width 0.508) (layer "B.Cu") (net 35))
 (segment (start 170.86 63.6) (end 175.94 58.52) (width 0.508) (layer "B.Cu") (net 35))
 (segment (start 150.54 50.9) (end 183.56 50.9) (width 0.508) (layer "B.Cu") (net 36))
 (segment (start 169.644 69.896) (end 169.644 71.723684) (width 0.508) (layer "B.Cu") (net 36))
 (segment (start 169.644 71.723684) (end 170.356316 72.436) (width 0.508) (layer "B.Cu") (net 36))
 (segment (start 188.64 55.98) (end 188.64 63.6) (width 0.508) (layer "B.Cu") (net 36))
 (segment (start 183.56 50.9) (end 188.64 55.98) (width 0.508) (layer "B.Cu") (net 36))
 (segment (start 170.356316 72.436) (end 179.804 72.436) (width 0.508) (layer "B.Cu") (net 36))
 (segment (start 170.86 68.68) (end 169.644 69.896) (width 0.508) (layer "B.Cu") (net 36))
 (segment (start 179.804 72.436) (end 188.64 63.6) (width 0.508) (layer "B.Cu") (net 36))
 (segment (start 145.46 55.98) (end 150.54 50.9) (width 0.508) (layer "B.Cu") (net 36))
 (segment (start 183.56 58.52) (end 181.02 55.98) (width 0.508) (layer "B.Cu") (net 37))
 (segment (start 170.86 71.22) (end 175.94 71.22) (width 0.508) (layer "B.Cu") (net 37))
 (segment (start 175.94 71.22) (end 183.56 63.6) (width 0.508) (layer "B.Cu") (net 37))
 (segment (start 183.56 63.6) (end 183.56 58.52) (width 0.508) (layer "B.Cu") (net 37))
 (segment (start 155.62 66.14) (end 145.46 76.3) (width 0.508) (layer "B.Cu") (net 33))
 (segment (start 155.62 58.52) (end 155.62 66.14) (width 0.508) (layer "B.Cu") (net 33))
 (segment (start 158.16 66.14) (end 158.16 58.52) (width 0.508) (layer "B.Cu") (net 32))
 (segment (start 148 76.3) (end 158.16 66.14) (width 0.508) (layer "B.Cu") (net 32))
 (segment (start 142.92 76.3) (end 142.92 78.84) (width 0.508) (layer "B.Cu") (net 34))
 (segment (start 160.7 58.52) (end 160.7 66.14) (width 0.508) (layer "B.Cu") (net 34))
 (segment (start 158.16 78.84) (end 160.7 76.3) (width 0.508) (layer "B.Cu") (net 34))
 (segment (start 160.7 76.3) (end 160.7 66.14) (width 0.508) (layer "B.Cu") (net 34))
 (segment (start 142.92 78.84) (end 158.16 78.84) (width 0.508) (layer "B.Cu") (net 34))
 (segment (start 168.32 61.06) (end 186.1 61.06) (width 0.508) (layer "F.Cu") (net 31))
 (segment (start 160.7 68.68) (end 168.32 61.06) (width 0.508) (layer "F.Cu") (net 31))
 (segment (start 158.16 68.68) (end 160.7 68.68) (width 0.508) (layer "F.Cu") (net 31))
 (via (at 186.1 61.06) (size 1.1) (drill 0.6426) (layers "F.Cu" "B.Cu") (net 31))
 (via (at 158.16 68.68) (size 0.8) (drill 0.4) (layers "F.Cu" "B.Cu") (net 31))
 (segment (start 186.1 55.98) (end 186.1 61.06) (width 0.508) (layer "B.Cu") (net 31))
 (segment (start 183.56 53.44) (end 186.1 55.98) (width 0.508) (layer "B.Cu") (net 31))
 (segment (start 163.24 53.44) (end 183.56 53.44) (width 0.508) (layer "B.Cu") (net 31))
 (segment (start 150.54 76.3) (end 158.16 68.68) (width 0.508) (layer "B.Cu") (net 31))
 (segment (start 160.7 55.98) (end 163.24 53.44) (width 0.508) (layer "B.Cu") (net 31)))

